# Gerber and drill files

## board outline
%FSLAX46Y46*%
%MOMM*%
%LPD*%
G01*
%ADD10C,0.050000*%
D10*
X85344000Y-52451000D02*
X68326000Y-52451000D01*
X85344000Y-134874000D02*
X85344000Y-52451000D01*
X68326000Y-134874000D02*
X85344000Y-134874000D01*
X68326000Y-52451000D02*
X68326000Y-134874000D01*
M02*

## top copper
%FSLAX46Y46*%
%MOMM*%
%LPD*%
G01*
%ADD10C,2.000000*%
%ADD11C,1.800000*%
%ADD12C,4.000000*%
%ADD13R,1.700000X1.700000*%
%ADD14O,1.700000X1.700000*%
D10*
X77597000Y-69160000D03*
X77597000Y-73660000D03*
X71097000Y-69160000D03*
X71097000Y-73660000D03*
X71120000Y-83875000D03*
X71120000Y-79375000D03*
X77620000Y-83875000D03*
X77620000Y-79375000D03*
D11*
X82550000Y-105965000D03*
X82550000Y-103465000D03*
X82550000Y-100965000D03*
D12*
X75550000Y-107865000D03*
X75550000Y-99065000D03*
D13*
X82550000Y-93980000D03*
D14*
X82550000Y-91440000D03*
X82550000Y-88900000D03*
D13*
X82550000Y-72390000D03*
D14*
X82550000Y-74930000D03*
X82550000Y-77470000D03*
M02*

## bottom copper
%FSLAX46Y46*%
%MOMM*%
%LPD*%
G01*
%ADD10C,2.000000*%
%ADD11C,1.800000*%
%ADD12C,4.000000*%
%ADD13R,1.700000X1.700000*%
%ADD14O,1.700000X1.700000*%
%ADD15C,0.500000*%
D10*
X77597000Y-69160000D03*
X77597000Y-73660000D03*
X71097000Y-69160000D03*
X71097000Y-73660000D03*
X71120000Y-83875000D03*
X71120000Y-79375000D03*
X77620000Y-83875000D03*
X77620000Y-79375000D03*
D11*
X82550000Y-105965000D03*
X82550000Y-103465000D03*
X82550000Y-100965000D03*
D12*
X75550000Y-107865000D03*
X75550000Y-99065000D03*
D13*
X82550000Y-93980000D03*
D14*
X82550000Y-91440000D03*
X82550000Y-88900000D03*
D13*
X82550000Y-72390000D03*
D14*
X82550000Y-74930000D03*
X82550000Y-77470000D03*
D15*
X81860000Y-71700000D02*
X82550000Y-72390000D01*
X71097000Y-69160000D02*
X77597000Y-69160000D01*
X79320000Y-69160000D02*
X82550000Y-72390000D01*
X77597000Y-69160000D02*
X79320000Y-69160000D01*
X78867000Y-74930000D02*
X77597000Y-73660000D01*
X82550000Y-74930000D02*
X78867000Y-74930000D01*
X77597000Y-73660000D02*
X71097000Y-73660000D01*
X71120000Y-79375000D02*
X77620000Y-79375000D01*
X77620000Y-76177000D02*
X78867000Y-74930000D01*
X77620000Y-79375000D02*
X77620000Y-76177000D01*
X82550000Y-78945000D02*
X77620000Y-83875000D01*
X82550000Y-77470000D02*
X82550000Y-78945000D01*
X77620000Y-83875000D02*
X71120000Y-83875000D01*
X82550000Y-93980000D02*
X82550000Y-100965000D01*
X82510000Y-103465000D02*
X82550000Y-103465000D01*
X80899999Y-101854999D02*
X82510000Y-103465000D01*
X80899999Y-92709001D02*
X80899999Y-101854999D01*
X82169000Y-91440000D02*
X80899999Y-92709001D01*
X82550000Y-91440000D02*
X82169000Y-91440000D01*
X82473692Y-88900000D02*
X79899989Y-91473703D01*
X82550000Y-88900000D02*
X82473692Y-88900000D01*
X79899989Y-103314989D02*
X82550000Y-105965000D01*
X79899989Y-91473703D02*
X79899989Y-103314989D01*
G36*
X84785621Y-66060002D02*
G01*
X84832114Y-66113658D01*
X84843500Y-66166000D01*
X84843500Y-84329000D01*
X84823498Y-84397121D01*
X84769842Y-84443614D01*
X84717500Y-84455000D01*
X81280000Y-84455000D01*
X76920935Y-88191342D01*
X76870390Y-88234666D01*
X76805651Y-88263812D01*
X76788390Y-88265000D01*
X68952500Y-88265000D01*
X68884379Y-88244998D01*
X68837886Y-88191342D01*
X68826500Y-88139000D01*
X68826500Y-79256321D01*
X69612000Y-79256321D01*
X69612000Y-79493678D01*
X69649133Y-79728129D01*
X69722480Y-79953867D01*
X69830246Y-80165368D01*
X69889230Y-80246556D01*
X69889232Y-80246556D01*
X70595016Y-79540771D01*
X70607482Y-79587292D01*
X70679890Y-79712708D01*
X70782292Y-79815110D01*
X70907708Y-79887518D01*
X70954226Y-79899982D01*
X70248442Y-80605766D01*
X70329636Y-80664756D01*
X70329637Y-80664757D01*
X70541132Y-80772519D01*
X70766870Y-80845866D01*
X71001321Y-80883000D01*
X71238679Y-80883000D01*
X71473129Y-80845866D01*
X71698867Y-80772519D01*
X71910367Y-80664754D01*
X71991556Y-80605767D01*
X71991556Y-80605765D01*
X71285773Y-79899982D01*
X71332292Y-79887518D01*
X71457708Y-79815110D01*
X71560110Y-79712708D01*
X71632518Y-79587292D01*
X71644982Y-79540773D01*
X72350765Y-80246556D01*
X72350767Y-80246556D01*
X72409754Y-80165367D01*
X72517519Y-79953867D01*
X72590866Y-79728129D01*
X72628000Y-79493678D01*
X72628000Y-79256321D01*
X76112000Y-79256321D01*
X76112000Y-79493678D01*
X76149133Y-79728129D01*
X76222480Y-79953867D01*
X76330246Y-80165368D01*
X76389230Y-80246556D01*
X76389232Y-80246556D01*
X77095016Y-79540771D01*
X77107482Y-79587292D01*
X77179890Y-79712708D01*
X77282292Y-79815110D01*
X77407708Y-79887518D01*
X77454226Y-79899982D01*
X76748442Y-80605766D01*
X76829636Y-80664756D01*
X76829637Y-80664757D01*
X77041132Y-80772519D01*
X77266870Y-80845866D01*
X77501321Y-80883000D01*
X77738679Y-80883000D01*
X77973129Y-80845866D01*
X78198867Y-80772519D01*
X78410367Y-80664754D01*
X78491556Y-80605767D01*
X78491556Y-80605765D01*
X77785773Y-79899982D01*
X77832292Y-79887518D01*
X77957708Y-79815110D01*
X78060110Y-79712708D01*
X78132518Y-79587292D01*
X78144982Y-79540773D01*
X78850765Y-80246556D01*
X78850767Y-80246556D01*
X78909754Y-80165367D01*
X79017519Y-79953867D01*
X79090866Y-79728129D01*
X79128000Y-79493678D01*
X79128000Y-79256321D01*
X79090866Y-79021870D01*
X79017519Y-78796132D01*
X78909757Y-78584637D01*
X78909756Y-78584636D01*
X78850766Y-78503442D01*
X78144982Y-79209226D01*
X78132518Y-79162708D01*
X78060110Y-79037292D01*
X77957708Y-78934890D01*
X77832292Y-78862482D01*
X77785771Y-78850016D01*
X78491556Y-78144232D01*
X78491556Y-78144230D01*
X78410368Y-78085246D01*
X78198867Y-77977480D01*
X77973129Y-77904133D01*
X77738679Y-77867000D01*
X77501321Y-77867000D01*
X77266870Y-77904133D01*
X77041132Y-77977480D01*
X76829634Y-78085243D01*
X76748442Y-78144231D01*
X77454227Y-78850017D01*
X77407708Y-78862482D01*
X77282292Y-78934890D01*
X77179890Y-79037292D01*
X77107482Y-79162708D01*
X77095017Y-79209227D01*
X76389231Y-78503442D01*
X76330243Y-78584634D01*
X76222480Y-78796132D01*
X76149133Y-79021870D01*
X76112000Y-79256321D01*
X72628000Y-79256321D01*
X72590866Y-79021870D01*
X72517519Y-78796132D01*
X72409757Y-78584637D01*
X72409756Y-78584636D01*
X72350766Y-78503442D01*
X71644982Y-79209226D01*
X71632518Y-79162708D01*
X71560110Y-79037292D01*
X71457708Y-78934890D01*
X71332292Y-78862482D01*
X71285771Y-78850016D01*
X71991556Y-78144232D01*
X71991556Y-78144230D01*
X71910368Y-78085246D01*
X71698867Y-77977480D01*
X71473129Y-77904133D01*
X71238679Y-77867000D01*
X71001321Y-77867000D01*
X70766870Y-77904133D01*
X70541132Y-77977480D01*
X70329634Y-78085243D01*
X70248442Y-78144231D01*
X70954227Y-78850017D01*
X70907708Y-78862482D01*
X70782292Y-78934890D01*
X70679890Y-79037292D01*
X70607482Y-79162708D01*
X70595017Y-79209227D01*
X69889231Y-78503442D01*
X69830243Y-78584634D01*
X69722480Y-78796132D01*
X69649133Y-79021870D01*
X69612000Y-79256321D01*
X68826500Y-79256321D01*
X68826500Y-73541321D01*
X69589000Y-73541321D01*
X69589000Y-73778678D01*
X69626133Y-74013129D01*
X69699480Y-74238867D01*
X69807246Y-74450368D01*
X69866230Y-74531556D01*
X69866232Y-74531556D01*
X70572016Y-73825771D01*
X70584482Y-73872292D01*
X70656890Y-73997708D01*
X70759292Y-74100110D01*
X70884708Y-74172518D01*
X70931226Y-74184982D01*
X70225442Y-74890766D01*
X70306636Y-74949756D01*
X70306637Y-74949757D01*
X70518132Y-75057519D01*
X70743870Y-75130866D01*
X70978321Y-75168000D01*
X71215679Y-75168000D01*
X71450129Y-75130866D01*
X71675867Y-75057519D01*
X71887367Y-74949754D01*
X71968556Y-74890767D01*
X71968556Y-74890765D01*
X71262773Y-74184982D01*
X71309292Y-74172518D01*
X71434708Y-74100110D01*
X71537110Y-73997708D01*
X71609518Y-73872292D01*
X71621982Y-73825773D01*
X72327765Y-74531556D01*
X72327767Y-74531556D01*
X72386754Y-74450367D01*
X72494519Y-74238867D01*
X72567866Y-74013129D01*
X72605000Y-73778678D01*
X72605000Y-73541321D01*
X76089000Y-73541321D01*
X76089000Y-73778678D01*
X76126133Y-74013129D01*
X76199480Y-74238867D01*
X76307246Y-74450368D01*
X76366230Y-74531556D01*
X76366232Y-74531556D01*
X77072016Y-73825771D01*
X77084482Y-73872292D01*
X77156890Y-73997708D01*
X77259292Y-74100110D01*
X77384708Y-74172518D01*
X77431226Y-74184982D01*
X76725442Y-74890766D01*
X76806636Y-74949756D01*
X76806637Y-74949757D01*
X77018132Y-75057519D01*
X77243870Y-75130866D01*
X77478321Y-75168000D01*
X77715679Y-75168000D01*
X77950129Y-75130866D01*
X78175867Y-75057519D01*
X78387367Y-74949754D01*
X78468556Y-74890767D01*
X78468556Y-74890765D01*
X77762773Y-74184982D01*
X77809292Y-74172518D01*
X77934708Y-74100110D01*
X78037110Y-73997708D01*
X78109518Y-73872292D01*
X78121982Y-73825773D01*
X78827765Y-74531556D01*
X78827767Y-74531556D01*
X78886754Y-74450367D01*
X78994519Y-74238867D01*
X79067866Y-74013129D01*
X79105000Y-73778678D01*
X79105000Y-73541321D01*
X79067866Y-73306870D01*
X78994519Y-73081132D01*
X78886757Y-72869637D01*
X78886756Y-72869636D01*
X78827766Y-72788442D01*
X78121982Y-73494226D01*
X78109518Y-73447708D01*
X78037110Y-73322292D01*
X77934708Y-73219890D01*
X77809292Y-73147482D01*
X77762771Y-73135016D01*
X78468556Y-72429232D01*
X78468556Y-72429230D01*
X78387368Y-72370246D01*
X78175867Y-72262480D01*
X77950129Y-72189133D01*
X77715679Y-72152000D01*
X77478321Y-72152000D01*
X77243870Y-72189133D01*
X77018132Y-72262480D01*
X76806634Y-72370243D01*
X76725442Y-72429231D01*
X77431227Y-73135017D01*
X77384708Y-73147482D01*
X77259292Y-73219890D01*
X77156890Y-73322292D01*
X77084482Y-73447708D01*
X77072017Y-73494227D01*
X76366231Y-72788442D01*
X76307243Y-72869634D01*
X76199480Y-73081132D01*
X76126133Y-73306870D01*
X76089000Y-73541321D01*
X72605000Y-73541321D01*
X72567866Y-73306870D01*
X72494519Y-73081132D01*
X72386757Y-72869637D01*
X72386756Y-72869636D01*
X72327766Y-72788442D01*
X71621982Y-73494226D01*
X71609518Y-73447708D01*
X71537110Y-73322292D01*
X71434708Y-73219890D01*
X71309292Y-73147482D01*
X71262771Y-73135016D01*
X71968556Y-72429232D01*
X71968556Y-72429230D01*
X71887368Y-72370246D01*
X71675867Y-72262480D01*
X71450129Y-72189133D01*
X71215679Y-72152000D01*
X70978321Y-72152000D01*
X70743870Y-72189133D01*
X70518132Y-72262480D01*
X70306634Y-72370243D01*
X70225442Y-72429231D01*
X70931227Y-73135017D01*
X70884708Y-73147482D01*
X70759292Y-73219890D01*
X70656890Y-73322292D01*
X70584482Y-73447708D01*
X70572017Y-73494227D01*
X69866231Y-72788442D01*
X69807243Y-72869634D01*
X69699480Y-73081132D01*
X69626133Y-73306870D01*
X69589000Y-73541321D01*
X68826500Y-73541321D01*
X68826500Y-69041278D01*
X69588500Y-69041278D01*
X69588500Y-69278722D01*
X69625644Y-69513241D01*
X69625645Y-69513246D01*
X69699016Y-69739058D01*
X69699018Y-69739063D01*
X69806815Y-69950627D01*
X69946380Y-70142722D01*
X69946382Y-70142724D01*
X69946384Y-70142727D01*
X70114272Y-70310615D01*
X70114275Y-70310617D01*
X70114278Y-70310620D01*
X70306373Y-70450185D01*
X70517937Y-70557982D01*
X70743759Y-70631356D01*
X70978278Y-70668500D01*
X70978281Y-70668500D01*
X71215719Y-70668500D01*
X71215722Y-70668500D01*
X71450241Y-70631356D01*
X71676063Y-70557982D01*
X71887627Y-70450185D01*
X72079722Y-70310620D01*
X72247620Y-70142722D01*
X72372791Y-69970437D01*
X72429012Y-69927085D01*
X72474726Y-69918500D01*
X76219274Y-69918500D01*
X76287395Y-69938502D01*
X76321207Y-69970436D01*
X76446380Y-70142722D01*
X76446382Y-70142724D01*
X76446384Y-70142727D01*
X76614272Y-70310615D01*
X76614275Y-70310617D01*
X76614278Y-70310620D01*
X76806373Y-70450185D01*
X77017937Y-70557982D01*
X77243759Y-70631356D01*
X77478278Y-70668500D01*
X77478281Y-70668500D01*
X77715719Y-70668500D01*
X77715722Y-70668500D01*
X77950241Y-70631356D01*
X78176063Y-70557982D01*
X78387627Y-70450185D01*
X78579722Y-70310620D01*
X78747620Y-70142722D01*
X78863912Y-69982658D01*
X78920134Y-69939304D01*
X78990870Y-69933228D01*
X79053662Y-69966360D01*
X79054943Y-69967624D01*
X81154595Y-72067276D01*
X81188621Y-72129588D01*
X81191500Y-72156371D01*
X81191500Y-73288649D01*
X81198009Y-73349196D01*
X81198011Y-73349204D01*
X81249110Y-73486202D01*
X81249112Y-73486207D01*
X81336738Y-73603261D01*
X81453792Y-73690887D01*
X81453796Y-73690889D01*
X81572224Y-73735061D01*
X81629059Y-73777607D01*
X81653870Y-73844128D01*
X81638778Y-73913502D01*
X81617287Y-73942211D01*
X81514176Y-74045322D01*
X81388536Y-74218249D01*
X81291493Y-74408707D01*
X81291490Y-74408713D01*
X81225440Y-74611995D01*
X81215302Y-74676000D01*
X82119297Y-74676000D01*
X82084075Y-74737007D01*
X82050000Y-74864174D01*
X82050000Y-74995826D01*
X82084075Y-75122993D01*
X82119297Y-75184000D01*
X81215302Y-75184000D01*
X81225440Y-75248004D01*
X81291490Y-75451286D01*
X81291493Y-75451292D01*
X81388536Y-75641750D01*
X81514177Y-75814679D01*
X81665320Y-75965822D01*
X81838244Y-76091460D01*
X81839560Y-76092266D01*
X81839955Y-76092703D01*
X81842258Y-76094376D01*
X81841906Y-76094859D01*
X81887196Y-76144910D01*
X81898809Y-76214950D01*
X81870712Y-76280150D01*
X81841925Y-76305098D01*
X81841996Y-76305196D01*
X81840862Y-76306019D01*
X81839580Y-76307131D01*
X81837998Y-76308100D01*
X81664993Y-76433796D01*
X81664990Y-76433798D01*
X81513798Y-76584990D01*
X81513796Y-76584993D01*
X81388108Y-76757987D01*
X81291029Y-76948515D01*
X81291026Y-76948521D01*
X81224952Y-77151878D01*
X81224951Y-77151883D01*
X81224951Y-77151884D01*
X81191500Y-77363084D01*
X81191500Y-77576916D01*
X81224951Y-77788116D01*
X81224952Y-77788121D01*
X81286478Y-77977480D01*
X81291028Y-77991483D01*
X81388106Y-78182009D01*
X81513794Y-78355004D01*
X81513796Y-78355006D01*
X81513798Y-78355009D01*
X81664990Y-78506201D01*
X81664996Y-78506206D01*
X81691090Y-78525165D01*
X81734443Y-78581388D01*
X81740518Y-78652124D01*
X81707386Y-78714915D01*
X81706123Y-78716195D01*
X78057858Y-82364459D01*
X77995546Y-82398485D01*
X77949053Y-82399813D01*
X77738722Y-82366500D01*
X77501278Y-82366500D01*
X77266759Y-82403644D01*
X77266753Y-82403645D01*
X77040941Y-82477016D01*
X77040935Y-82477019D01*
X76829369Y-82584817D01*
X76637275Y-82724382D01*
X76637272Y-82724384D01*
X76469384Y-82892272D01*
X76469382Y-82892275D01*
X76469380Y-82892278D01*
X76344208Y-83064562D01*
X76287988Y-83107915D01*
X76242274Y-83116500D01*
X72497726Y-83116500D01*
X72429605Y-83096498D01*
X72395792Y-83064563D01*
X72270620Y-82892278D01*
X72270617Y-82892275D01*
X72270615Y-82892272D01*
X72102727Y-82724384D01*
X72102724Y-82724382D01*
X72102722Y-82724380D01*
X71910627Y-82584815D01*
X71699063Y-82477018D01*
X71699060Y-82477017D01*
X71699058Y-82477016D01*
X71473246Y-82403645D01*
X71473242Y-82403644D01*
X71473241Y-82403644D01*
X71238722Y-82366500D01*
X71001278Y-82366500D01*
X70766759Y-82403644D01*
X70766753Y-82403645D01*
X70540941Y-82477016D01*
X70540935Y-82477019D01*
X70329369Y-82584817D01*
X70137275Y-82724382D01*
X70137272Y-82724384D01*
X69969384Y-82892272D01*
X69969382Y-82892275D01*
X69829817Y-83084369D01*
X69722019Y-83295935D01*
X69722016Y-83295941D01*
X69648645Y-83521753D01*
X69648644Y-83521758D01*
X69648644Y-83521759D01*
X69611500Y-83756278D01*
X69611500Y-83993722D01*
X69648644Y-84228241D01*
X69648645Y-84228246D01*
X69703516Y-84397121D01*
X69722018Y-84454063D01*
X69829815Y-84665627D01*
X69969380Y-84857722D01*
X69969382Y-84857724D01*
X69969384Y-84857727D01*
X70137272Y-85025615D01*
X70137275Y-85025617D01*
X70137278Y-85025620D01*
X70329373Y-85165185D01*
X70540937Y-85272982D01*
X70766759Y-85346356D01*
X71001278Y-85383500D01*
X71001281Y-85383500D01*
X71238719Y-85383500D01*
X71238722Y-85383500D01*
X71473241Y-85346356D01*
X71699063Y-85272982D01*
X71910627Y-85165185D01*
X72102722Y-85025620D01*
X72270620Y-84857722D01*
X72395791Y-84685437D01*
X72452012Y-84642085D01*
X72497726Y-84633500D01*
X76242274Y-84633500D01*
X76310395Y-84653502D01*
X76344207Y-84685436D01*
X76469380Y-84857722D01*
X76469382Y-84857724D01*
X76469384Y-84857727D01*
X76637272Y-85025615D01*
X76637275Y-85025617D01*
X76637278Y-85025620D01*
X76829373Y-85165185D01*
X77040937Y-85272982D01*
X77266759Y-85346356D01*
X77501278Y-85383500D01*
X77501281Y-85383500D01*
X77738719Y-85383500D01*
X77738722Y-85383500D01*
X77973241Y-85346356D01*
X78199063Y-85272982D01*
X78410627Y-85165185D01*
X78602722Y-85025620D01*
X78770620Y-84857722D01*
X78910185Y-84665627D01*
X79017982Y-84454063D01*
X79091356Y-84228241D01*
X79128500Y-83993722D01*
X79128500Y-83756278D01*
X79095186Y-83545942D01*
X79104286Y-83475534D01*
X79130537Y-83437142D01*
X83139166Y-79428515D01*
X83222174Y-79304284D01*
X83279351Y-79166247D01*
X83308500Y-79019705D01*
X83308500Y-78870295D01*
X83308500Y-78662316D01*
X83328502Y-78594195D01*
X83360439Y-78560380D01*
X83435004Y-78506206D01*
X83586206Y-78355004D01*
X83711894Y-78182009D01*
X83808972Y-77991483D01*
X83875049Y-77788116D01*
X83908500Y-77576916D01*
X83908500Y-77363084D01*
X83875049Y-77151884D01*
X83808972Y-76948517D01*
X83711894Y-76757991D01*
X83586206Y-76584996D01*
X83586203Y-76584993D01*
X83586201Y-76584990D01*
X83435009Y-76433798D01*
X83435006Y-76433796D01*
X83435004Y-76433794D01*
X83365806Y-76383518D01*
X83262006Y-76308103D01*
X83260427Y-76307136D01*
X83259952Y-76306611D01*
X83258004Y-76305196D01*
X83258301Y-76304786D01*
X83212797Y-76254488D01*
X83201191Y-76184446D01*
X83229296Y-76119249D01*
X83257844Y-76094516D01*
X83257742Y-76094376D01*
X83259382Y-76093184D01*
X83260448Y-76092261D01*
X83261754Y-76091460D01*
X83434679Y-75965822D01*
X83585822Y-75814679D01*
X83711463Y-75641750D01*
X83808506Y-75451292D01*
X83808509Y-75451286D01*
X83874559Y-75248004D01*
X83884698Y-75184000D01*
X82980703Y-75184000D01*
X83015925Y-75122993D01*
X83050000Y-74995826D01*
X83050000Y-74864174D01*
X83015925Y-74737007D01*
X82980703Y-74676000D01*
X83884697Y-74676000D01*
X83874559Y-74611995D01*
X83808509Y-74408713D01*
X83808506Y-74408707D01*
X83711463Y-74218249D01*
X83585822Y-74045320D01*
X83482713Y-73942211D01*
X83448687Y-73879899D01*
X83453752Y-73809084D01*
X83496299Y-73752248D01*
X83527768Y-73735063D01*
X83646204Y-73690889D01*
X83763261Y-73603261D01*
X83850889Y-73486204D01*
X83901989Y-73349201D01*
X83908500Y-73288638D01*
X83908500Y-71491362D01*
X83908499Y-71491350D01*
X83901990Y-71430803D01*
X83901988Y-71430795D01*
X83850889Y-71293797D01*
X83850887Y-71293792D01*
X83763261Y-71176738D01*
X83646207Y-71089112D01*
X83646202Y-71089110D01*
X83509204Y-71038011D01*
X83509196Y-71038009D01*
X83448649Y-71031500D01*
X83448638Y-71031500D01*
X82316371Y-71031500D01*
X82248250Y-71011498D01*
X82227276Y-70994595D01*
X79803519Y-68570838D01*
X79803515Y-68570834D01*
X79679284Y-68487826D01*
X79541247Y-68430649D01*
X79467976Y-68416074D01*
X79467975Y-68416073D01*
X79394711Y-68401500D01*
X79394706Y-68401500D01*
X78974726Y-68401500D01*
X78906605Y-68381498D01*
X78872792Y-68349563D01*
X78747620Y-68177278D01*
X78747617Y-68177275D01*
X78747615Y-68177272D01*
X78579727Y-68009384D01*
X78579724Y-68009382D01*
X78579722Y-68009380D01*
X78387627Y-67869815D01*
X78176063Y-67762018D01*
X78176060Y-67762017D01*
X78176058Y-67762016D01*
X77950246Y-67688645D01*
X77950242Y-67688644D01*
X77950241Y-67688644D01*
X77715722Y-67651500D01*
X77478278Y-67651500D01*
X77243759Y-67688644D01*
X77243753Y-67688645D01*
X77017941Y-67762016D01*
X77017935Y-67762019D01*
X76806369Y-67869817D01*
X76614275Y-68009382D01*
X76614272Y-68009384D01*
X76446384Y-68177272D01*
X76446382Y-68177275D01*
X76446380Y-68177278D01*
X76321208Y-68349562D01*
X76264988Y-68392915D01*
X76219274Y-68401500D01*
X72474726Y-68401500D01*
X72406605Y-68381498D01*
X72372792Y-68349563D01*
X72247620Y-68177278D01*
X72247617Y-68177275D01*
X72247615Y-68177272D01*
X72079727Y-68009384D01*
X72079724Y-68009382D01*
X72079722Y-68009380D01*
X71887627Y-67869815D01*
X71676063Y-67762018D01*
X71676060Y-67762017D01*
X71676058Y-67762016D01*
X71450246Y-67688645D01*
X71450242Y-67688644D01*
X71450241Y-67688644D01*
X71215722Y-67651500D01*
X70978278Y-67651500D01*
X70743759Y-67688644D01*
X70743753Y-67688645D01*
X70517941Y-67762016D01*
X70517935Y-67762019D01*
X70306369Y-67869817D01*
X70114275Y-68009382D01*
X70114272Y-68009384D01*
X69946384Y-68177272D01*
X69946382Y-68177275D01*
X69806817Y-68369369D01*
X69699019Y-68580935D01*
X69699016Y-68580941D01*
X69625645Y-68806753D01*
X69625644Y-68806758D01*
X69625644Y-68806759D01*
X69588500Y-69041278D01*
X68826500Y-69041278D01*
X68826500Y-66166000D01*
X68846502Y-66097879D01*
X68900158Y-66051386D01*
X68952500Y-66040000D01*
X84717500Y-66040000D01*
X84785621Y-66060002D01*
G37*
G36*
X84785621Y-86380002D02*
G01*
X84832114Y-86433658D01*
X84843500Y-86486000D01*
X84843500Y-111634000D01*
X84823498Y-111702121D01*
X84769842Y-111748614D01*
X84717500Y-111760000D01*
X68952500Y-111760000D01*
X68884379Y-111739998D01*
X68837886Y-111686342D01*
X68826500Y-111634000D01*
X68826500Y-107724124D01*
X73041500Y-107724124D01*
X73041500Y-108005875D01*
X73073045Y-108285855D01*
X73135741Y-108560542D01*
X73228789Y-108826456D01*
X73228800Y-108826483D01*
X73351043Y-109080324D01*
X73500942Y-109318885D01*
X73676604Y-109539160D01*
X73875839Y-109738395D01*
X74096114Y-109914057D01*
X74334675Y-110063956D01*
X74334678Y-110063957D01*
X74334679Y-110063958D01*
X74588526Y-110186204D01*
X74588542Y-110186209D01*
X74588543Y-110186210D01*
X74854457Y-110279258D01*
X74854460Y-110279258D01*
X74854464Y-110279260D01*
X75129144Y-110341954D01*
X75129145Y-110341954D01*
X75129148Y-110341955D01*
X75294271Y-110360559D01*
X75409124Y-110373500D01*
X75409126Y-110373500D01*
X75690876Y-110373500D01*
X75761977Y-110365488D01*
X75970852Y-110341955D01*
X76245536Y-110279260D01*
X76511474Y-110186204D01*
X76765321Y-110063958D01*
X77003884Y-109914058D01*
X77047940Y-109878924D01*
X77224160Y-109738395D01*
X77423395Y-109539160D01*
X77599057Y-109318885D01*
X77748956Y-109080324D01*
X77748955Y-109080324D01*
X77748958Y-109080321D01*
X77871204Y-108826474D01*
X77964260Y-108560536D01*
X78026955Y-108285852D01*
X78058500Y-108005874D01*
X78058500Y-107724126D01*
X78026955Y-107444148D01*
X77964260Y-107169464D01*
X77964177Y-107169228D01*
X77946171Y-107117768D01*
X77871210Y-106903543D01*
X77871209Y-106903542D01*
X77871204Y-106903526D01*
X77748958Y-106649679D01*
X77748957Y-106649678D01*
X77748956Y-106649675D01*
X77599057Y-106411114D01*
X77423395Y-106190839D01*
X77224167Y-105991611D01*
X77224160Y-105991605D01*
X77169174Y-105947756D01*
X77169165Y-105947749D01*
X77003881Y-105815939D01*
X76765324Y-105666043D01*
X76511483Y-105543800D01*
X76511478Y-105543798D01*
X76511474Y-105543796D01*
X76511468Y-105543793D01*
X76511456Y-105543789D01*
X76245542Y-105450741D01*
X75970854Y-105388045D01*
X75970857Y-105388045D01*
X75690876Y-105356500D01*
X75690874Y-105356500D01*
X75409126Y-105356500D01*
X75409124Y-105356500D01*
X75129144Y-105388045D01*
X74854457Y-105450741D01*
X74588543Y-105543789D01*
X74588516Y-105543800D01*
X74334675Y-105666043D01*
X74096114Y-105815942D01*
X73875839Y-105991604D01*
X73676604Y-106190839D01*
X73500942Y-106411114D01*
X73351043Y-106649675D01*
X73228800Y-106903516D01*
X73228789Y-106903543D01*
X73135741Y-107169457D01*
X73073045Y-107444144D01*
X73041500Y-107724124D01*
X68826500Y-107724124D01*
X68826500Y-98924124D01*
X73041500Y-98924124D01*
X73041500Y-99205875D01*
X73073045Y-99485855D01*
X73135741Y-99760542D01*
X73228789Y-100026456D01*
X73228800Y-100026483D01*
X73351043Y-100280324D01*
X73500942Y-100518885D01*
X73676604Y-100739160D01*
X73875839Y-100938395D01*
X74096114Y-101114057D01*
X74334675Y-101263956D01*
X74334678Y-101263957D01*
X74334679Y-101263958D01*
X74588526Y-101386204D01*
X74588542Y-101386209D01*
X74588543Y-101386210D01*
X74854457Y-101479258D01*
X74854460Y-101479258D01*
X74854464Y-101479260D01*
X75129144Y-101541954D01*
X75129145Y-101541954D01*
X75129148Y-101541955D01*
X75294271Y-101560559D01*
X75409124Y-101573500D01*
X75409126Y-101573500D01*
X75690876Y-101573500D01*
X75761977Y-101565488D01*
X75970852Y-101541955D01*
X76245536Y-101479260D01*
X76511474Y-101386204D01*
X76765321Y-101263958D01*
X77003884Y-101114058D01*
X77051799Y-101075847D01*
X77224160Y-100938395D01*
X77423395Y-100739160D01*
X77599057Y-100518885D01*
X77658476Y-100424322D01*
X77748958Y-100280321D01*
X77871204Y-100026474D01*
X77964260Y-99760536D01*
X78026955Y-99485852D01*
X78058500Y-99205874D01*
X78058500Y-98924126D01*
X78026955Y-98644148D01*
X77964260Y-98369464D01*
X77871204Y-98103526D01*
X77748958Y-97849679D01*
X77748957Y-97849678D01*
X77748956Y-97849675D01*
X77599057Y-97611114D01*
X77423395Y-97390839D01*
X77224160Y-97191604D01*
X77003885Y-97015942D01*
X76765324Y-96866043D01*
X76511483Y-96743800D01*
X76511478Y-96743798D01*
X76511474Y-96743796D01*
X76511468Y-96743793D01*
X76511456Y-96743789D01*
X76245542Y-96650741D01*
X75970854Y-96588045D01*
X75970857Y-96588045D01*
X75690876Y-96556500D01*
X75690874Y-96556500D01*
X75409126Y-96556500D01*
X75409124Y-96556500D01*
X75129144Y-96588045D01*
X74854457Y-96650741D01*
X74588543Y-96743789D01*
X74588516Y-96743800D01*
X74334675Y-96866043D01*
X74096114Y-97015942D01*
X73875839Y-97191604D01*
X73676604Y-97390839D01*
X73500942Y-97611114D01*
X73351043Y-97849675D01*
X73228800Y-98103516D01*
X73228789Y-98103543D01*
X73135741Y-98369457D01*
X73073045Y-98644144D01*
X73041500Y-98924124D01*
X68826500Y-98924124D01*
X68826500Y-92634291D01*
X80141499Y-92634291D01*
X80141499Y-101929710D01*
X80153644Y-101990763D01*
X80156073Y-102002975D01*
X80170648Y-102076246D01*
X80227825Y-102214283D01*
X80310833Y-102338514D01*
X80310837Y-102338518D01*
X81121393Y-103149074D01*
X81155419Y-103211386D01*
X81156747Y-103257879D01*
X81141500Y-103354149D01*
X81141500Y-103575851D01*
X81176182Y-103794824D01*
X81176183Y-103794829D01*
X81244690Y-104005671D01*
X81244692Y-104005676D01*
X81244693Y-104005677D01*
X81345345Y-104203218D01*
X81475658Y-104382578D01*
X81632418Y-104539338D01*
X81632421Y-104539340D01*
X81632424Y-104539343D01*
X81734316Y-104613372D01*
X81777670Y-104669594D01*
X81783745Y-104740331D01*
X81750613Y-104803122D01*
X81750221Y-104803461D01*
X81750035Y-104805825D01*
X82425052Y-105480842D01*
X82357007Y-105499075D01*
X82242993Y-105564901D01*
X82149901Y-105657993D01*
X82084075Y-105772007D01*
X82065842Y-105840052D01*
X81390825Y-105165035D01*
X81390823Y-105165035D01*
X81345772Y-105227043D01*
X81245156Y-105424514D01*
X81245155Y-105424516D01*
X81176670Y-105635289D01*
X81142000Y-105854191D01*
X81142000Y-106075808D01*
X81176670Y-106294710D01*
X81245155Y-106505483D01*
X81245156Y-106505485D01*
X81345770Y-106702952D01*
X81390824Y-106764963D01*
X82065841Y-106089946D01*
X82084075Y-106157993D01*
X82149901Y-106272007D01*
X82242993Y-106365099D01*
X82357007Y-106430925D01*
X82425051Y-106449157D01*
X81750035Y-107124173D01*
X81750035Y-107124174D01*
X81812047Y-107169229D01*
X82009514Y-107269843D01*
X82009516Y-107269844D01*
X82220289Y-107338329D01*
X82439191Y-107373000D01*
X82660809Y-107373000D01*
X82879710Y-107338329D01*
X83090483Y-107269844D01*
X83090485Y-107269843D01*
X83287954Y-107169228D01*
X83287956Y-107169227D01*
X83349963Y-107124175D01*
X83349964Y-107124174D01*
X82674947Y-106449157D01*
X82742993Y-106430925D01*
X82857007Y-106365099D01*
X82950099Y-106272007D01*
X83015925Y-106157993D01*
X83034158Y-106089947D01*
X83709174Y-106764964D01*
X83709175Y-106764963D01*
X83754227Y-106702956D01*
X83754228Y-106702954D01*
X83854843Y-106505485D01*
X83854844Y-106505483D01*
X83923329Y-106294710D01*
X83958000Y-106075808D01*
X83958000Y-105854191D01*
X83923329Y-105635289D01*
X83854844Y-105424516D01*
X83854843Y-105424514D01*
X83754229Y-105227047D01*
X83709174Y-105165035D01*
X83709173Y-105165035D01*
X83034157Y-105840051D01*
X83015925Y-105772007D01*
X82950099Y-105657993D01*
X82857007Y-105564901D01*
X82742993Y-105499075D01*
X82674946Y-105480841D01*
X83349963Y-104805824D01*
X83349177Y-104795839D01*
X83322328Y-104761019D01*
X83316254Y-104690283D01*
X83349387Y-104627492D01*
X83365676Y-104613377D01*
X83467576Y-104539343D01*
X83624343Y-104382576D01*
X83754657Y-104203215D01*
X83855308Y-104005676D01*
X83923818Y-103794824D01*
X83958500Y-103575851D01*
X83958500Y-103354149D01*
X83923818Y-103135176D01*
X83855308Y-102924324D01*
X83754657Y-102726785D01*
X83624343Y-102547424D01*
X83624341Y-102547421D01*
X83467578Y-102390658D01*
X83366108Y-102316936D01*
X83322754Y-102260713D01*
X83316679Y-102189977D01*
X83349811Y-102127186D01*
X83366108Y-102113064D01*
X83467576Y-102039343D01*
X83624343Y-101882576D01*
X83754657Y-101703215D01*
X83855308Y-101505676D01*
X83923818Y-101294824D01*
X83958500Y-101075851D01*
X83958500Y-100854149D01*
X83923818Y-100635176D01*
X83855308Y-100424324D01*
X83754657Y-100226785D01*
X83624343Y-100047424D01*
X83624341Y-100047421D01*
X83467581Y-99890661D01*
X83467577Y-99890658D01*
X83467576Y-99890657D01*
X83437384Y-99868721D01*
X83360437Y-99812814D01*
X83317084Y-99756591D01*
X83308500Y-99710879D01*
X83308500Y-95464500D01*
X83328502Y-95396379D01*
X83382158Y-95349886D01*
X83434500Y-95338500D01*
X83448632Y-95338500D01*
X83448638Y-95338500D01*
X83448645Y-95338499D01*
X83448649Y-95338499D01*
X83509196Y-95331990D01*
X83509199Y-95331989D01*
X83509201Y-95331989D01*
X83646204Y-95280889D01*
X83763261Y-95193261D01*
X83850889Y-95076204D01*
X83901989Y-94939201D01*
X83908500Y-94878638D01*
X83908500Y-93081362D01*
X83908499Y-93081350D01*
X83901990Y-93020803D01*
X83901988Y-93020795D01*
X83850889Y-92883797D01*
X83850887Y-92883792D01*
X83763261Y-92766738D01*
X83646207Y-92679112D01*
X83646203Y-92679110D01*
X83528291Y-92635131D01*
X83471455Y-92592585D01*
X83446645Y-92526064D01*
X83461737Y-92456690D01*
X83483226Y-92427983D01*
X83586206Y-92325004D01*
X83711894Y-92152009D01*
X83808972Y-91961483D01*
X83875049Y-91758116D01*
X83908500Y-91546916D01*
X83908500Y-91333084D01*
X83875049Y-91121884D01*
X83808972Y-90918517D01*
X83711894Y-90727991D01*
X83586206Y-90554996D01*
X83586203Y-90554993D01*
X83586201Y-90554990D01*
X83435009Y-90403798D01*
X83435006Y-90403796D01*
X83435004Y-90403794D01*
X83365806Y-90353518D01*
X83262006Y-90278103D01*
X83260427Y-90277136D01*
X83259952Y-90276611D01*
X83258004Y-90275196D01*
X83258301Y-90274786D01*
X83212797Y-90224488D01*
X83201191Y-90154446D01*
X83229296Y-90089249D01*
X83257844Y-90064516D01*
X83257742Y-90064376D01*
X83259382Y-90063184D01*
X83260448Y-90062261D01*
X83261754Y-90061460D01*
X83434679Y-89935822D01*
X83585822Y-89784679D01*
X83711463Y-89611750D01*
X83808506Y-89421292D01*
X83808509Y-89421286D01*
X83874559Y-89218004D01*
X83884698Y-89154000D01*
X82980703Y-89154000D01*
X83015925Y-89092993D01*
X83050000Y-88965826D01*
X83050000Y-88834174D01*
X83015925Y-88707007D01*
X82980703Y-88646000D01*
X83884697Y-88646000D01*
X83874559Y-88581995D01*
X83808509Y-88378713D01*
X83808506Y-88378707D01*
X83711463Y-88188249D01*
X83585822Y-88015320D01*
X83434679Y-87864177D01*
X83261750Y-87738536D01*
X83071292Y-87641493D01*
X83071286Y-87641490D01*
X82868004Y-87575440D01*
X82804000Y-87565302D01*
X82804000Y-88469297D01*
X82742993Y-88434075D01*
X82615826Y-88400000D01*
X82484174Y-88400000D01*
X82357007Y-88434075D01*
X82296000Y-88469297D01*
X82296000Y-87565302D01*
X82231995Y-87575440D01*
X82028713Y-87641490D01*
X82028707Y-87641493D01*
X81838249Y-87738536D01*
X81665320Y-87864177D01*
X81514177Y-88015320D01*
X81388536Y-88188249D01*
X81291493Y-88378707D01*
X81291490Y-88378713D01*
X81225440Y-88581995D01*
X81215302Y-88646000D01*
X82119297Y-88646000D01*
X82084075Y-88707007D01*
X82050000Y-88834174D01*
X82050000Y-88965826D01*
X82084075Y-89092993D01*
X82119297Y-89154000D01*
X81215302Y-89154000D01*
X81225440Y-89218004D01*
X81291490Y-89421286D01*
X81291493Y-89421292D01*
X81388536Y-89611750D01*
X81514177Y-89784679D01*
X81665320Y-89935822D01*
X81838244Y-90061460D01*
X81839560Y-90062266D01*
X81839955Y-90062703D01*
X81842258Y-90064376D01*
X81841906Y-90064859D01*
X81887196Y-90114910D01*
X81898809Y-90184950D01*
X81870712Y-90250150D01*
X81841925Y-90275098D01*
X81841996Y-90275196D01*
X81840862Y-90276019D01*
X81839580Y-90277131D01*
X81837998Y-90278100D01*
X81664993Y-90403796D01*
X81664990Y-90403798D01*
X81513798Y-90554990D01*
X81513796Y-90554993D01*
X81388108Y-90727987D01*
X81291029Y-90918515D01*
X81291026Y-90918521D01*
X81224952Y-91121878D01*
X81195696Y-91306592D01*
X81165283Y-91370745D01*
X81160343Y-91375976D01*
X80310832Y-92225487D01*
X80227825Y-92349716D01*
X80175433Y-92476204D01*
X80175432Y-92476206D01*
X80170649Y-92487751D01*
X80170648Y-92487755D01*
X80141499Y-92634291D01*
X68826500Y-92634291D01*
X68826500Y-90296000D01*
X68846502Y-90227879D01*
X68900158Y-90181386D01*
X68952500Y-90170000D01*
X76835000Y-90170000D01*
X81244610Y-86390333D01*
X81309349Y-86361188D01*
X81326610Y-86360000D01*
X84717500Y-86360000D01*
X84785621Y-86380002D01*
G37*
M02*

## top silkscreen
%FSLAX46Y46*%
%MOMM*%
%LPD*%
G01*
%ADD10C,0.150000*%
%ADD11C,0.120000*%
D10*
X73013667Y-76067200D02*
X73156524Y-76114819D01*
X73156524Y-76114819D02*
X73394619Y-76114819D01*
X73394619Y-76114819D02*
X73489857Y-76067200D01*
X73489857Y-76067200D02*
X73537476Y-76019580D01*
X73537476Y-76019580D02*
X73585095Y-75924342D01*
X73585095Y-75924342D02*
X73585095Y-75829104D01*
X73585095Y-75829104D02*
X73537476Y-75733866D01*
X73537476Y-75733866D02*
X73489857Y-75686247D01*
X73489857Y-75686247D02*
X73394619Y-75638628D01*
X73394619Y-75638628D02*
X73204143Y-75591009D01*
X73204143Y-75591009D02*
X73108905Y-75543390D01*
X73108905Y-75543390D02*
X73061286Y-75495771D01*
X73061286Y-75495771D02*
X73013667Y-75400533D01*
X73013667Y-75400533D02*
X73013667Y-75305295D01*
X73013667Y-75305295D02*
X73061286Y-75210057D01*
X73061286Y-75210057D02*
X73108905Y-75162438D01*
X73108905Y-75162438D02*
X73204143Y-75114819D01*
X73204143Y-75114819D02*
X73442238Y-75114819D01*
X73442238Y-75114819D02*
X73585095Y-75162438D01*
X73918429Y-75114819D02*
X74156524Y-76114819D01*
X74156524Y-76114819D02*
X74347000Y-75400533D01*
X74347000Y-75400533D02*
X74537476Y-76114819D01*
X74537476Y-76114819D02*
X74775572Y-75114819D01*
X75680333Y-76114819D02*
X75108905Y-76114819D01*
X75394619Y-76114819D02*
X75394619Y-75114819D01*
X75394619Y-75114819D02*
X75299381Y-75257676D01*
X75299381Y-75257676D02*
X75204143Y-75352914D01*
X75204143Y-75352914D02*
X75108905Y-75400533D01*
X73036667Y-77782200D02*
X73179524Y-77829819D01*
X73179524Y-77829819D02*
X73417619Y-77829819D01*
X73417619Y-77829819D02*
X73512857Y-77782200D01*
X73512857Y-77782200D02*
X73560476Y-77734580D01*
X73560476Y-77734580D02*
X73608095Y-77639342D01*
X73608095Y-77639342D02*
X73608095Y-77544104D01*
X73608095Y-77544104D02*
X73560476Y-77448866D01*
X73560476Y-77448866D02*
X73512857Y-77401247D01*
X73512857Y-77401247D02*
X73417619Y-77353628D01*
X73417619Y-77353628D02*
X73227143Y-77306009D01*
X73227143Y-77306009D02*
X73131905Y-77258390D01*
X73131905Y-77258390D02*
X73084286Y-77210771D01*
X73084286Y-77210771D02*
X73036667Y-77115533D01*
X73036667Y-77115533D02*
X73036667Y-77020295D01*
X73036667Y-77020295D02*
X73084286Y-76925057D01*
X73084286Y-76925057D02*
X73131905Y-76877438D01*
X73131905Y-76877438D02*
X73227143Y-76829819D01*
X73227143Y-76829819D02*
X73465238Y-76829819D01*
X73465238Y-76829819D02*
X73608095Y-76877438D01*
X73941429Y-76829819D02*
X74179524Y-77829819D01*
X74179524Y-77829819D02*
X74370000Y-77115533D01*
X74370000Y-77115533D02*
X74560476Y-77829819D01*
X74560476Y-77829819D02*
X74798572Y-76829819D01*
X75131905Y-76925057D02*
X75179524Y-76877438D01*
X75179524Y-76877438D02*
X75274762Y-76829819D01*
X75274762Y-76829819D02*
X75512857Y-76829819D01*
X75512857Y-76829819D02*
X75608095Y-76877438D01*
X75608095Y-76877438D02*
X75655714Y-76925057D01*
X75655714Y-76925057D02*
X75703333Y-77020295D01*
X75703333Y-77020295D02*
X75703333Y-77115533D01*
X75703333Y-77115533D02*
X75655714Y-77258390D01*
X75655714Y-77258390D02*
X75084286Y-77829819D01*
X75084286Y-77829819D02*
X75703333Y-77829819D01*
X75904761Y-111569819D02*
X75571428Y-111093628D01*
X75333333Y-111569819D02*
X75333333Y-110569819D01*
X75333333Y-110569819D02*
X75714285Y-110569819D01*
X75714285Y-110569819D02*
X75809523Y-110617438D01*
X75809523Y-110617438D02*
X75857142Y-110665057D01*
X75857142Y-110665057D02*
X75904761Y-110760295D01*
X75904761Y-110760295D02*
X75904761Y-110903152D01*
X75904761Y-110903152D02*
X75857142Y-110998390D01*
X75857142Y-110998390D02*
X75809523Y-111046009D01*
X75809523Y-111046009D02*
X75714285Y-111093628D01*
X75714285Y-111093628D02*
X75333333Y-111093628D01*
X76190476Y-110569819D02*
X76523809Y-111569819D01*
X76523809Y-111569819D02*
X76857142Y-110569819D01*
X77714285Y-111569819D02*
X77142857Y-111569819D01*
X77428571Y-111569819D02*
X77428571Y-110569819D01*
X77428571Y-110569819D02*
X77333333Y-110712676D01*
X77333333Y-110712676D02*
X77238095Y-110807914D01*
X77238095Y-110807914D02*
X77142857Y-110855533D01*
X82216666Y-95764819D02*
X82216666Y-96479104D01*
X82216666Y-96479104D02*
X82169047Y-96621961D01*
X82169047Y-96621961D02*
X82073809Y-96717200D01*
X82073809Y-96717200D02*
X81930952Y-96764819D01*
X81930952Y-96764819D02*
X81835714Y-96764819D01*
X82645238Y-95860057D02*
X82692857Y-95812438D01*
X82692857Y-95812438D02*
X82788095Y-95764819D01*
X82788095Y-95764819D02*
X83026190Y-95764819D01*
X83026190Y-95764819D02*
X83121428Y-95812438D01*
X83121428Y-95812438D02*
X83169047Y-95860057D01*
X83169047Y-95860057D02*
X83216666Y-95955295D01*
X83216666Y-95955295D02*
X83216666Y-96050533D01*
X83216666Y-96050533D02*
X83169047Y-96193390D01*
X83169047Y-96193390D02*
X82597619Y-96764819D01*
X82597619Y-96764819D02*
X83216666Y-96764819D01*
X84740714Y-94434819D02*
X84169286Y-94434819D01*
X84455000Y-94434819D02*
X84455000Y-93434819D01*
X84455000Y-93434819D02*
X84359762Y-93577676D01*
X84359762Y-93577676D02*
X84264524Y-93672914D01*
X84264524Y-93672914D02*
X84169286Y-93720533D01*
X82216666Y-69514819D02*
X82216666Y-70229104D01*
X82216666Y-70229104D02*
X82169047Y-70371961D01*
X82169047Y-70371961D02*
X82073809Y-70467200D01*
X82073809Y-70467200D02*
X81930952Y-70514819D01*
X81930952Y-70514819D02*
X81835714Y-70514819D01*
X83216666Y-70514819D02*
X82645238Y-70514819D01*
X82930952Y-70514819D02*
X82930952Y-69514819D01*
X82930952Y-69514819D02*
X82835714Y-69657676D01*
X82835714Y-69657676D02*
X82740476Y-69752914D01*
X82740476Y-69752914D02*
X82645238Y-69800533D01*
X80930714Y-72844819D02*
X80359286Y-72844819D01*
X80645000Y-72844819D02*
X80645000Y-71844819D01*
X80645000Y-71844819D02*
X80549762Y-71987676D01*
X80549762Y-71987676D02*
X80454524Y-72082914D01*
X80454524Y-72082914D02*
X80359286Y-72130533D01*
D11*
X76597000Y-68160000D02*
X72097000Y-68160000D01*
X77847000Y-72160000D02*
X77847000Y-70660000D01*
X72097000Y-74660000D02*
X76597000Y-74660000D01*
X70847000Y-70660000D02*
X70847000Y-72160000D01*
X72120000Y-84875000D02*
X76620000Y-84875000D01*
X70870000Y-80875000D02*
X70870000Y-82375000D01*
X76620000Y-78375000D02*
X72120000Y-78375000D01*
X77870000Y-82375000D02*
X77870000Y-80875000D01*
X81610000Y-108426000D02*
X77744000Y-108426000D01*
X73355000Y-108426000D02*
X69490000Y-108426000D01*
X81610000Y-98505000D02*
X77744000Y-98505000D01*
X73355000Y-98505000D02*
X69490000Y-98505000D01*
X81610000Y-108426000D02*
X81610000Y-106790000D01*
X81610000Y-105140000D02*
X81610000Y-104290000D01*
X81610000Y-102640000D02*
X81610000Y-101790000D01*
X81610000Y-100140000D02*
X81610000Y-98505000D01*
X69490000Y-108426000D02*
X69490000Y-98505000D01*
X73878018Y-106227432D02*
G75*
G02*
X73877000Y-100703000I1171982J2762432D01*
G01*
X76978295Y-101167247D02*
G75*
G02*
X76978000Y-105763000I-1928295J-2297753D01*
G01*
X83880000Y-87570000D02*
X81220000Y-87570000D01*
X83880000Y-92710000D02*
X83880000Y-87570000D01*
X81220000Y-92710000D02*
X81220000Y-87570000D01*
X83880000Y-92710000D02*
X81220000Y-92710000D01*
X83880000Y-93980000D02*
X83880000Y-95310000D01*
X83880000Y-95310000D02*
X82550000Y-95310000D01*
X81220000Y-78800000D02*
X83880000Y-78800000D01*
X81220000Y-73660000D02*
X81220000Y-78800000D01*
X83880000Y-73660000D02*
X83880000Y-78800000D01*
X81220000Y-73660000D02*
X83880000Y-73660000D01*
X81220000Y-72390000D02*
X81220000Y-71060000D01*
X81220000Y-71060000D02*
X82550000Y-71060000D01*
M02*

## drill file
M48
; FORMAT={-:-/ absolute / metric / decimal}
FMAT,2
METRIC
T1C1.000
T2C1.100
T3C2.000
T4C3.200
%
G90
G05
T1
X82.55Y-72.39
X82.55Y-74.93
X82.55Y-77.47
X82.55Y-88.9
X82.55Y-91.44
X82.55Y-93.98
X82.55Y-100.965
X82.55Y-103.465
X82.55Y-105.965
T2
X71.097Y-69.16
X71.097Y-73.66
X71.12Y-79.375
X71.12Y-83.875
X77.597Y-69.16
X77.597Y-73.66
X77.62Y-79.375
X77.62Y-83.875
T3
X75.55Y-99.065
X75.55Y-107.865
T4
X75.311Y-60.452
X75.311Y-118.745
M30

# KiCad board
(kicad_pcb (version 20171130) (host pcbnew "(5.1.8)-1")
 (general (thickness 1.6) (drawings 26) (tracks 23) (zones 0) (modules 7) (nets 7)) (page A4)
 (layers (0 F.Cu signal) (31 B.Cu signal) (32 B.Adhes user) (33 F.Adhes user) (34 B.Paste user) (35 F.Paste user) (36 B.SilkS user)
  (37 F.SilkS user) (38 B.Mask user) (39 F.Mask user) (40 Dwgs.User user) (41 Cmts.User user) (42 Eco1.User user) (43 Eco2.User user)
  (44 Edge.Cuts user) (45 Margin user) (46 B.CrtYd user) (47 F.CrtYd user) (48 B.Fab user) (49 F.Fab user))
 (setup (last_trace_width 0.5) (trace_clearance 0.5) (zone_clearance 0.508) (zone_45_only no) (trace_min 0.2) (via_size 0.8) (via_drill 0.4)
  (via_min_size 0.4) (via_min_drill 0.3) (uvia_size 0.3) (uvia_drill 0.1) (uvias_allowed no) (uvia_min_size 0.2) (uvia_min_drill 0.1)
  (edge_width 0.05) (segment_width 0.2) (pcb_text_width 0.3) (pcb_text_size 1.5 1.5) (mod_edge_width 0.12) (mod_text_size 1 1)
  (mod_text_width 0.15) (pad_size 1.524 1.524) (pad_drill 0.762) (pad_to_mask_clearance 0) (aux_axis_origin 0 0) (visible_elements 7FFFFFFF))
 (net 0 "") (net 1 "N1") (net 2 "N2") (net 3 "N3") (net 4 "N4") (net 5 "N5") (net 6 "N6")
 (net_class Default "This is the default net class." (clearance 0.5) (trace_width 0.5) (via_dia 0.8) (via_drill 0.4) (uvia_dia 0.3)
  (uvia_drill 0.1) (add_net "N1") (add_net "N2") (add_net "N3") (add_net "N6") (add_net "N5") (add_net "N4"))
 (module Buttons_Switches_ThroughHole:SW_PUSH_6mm (layer F.Cu) (at 77.597 73.66 180)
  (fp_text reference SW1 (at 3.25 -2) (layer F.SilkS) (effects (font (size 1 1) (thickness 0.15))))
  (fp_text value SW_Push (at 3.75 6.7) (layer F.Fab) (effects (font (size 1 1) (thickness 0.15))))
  (fp_line (start 1 5.5) (end 5.5 5.5) (layer F.SilkS) (width 0.12))
  (fp_line (start -0.25 1.5) (end -0.25 3) (layer F.SilkS) (width 0.12))
  (fp_line (start 5.5 -1) (end 1 -1) (layer F.SilkS) (width 0.12))
  (fp_line (start 6.75 3) (end 6.75 1.5) (layer F.SilkS) (width 0.12))
  (pad 2 thru_hole circle (at 0 4.5 270) (size 2 2) (drill 1.1) (layers *.Cu *.Mask) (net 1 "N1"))
  (pad 1 thru_hole circle (at 0 0 270) (size 2 2) (drill 1.1) (layers *.Cu *.Mask) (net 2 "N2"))
  (pad 2 thru_hole circle (at 6.5 4.5 270) (size 2 2) (drill 1.1) (layers *.Cu *.Mask) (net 1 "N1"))
  (pad 1 thru_hole circle (at 6.5 0 270) (size 2 2) (drill 1.1) (layers *.Cu *.Mask) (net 2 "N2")))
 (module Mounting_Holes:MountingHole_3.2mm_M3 (layer F.Cu) (at 75.311 118.745)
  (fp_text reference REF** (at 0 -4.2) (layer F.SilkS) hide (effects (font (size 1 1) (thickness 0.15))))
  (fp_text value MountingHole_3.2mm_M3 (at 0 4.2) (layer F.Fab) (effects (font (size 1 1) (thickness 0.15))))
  (pad 1 np_thru_hole circle (at 0 0) (size 3.2 3.2) (drill 3.2) (layers *.Cu *.Mask)))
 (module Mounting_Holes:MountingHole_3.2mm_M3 (layer F.Cu) (at 75.311 60.452)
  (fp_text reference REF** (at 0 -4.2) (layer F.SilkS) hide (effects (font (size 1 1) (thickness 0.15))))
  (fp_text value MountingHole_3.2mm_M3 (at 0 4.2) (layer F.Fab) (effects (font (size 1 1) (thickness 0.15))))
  (pad 1 np_thru_hole circle (at 0 0) (size 3.2 3.2) (drill 3.2) (layers *.Cu *.Mask)))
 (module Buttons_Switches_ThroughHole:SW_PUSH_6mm (layer F.Cu) (at 71.12 79.375)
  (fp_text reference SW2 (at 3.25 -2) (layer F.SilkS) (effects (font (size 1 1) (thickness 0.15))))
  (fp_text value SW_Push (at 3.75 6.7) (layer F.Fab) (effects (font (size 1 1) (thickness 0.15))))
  (fp_line (start 1 5.5) (end 5.5 5.5) (layer F.SilkS) (width 0.12))
  (fp_line (start -0.25 1.5) (end -0.25 3) (layer F.SilkS) (width 0.12))
  (fp_line (start 5.5 -1) (end 1 -1) (layer F.SilkS) (width 0.12))
  (fp_line (start 6.75 3) (end 6.75 1.5) (layer F.SilkS) (width 0.12))
  (pad 2 thru_hole circle (at 0 4.5 90) (size 2 2) (drill 1.1) (layers *.Cu *.Mask) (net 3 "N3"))
  (pad 1 thru_hole circle (at 0 0 90) (size 2 2) (drill 1.1) (layers *.Cu *.Mask) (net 2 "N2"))
  (pad 2 thru_hole circle (at 6.5 4.5 90) (size 2 2) (drill 1.1) (layers *.Cu *.Mask) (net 3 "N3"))
  (pad 1 thru_hole circle (at 6.5 0 90) (size 2 2) (drill 1.1) (layers *.Cu *.Mask) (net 2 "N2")))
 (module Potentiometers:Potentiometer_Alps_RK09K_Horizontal (layer F.Cu) (at 82.55 100.965 180)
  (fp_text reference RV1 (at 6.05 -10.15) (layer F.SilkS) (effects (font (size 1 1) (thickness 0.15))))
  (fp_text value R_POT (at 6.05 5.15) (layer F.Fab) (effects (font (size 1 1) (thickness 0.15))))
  (fp_line (start 0.94 -7.461) (end 4.806 -7.461) (layer F.SilkS) (width 0.12))
  (fp_line (start 9.195 -7.461) (end 13.06 -7.461) (layer F.SilkS) (width 0.12))
  (fp_line (start 0.94 2.46) (end 4.806 2.46) (layer F.SilkS) (width 0.12))
  (fp_line (start 9.195 2.46) (end 13.06 2.46) (layer F.SilkS) (width 0.12))
  (fp_line (start 0.94 -7.461) (end 0.94 -5.825) (layer F.SilkS) (width 0.12))
  (fp_line (start 0.94 -4.175) (end 0.94 -3.325) (layer F.SilkS) (width 0.12))
  (fp_line (start 0.94 -1.675) (end 0.94 -0.825) (layer F.SilkS) (width 0.12))
  (fp_line (start 0.94 0.825) (end 0.94 2.46) (layer F.SilkS) (width 0.12))
  (fp_line (start 13.06 -7.461) (end 13.06 2.46) (layer F.SilkS) (width 0.12))
  (fp_arc (start 7.5 -2.5) (end 8.673 0.262) (angle -134) (layer F.SilkS) (width 0.12))
  (fp_arc (start 7.5 -2.5) (end 5.572 -4.798) (angle -100) (layer F.SilkS) (width 0.12))
  (pad 3 thru_hole circle (at 0 -5 180) (size 1.8 1.8) (drill 1) (layers *.Cu *.Mask) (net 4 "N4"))
  (pad 2 thru_hole circle (at 0 -2.5 180) (size 1.8 1.8) (drill 1) (layers *.Cu *.Mask) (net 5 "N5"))
  (pad 1 thru_hole circle (at 0 0 180) (size 1.8 1.8) (drill 1) (layers *.Cu *.Mask) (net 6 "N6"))
  (pad 0 np_thru_hole circle (at 7 -6.9 180) (size 4 4) (drill 2) (layers *.Cu *.Mask))
  (pad 0 np_thru_hole circle (at 7 1.9 180) (size 4 4) (drill 2) (layers *.Cu *.Mask)))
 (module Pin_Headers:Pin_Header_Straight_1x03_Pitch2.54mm (layer F.Cu) (at 82.55 93.98 180)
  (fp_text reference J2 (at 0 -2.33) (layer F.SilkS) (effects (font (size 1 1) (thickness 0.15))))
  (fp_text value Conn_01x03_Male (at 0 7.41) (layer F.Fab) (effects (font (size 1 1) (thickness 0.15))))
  (fp_line (start -1.33 6.41) (end 1.33 6.41) (layer F.SilkS) (width 0.12))
  (fp_line (start -1.33 1.27) (end -1.33 6.41) (layer F.SilkS) (width 0.12))
  (fp_line (start 1.33 1.27) (end 1.33 6.41) (layer F.SilkS) (width 0.12))
  (fp_line (start -1.33 1.27) (end 1.33 1.27) (layer F.SilkS) (width 0.12))
  (fp_line (start -1.33 0) (end -1.33 -1.33) (layer F.SilkS) (width 0.12))
  (fp_line (start -1.33 -1.33) (end 0 -1.33) (layer F.SilkS) (width 0.12))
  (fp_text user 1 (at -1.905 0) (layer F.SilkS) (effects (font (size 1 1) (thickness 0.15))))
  (pad 1 thru_hole rect (at 0 0 180) (size 1.7 1.7) (drill 1) (layers *.Cu *.Mask) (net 6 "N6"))
  (pad 2 thru_hole oval (at 0 2.54 180) (size 1.7 1.7) (drill 1) (layers *.Cu *.Mask) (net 5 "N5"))
  (pad 3 thru_hole oval (at 0 5.08 180) (size 1.7 1.7) (drill 1) (layers *.Cu *.Mask) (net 4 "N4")))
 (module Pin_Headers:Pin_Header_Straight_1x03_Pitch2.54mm (layer F.Cu) (at 82.55 72.39)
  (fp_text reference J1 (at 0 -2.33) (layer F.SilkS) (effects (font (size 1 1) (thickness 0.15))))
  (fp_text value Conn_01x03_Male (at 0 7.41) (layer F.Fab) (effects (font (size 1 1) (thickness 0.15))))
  (fp_line (start -1.33 6.41) (end 1.33 6.41) (layer F.SilkS) (width 0.12))
  (fp_line (start -1.33 1.27) (end -1.33 6.41) (layer F.SilkS) (width 0.12))
  (fp_line (start 1.33 1.27) (end 1.33 6.41) (layer F.SilkS) (width 0.12))
  (fp_line (start -1.33 1.27) (end 1.33 1.27) (layer F.SilkS) (width 0.12))
  (fp_line (start -1.33 0) (end -1.33 -1.33) (layer F.SilkS) (width 0.12))
  (fp_line (start -1.33 -1.33) (end 0 -1.33) (layer F.SilkS) (width 0.12))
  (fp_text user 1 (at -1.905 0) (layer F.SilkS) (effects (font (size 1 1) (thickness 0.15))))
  (pad 1 thru_hole rect (at 0 0) (size 1.7 1.7) (drill 1) (layers *.Cu *.Mask) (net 1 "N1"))
  (pad 2 thru_hole oval (at 0 2.54) (size 1.7 1.7) (drill 1) (layers *.Cu *.Mask) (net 2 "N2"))
  (pad 3 thru_hole oval (at 0 5.08) (size 1.7 1.7) (drill 1) (layers *.Cu *.Mask) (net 3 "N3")))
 (gr_line (start 85.344 52.451) (end 68.326 52.451) (layer Edge.Cuts) (width 0.05))
 (gr_line (start 85.344 134.874) (end 85.344 52.451) (layer Edge.Cuts) (width 0.05))
 (gr_line (start 68.326 134.874) (end 85.344 134.874) (layer Edge.Cuts) (width 0.05))
 (gr_line (start 68.326 52.451) (end 68.326 134.874) (layer Edge.Cuts) (width 0.05))
 (segment (start 81.86 71.7) (end 82.55 72.39) (width 0.5) (layer B.Cu) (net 1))
 (segment (start 71.097 69.16) (end 77.597 69.16) (width 0.5) (layer B.Cu) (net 1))
 (segment (start 79.32 69.16) (end 82.55 72.39) (width 0.5) (layer B.Cu) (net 1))
 (segment (start 77.597 69.16) (end 79.32 69.16) (width 0.5) (layer B.Cu) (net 1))
 (segment (start 78.867 74.93) (end 77.597 73.66) (width 0.5) (layer B.Cu) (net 2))
 (segment (start 82.55 74.93) (end 78.867 74.93) (width 0.5) (layer B.Cu) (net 2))
 (segment (start 77.597 73.66) (end 71.097 73.66) (width 0.5) (layer B.Cu) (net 2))
 (segment (start 71.12 79.375) (end 77.62 79.375) (width 0.5) (layer B.Cu) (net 2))
 (segment (start 77.62 76.177) (end 78.867 74.93) (width 0.5) (layer B.Cu) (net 2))
 (segment (start 77.62 79.375) (end 77.62 76.177) (width 0.5) (layer B.Cu) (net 2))
 (segment (start 82.55 78.945) (end 77.62 83.875) (width 0.5) (layer B.Cu) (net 3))
 (segment (start 82.55 77.47) (end 82.55 78.945) (width 0.5) (layer B.Cu) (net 3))
 (segment (start 77.62 83.875) (end 71.12 83.875) (width 0.5) (layer B.Cu) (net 3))
 (segment (start 82.55 93.98) (end 82.55 100.965) (width 0.5) (layer B.Cu) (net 6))
 (segment (start 82.51 103.465) (end 82.55 103.465) (width 0.5) (layer B.Cu) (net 5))
 (segment (start 80.899999 101.854999) (end 82.51 103.465) (width 0.5) (layer B.Cu) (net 5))
 (segment (start 80.899999 92.709001) (end 80.899999 101.854999) (width 0.5) (layer B.Cu) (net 5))
 (segment (start 82.169 91.44) (end 80.899999 92.709001) (width 0.5) (layer B.Cu) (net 5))
 (segment (start 82.55 91.44) (end 82.169 91.44) (width 0.5) (layer B.Cu) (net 5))
 (segment (start 82.473692 88.9) (end 79.899989 91.473703) (width 0.5) (layer B.Cu) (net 4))
 (segment (start 82.55 88.9) (end 82.473692 88.9) (width 0.5) (layer B.Cu) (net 4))
 (segment (start 79.899989 103.314989) (end 82.55 105.965) (width 0.5) (layer B.Cu) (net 4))
 (segment (start 79.899989 91.473703) (end 79.899989 103.314989) (width 0.5) (layer B.Cu) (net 4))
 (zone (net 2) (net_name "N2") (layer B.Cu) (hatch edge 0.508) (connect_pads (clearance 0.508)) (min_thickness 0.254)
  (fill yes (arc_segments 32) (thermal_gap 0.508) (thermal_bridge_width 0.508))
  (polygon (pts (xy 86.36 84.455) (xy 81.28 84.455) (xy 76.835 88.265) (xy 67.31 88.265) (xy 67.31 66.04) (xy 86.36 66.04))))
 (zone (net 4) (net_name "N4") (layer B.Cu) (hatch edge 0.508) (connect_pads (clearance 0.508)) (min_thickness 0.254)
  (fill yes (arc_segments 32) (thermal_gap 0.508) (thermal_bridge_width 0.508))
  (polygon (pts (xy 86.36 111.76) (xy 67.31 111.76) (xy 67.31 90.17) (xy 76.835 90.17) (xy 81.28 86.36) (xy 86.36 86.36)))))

